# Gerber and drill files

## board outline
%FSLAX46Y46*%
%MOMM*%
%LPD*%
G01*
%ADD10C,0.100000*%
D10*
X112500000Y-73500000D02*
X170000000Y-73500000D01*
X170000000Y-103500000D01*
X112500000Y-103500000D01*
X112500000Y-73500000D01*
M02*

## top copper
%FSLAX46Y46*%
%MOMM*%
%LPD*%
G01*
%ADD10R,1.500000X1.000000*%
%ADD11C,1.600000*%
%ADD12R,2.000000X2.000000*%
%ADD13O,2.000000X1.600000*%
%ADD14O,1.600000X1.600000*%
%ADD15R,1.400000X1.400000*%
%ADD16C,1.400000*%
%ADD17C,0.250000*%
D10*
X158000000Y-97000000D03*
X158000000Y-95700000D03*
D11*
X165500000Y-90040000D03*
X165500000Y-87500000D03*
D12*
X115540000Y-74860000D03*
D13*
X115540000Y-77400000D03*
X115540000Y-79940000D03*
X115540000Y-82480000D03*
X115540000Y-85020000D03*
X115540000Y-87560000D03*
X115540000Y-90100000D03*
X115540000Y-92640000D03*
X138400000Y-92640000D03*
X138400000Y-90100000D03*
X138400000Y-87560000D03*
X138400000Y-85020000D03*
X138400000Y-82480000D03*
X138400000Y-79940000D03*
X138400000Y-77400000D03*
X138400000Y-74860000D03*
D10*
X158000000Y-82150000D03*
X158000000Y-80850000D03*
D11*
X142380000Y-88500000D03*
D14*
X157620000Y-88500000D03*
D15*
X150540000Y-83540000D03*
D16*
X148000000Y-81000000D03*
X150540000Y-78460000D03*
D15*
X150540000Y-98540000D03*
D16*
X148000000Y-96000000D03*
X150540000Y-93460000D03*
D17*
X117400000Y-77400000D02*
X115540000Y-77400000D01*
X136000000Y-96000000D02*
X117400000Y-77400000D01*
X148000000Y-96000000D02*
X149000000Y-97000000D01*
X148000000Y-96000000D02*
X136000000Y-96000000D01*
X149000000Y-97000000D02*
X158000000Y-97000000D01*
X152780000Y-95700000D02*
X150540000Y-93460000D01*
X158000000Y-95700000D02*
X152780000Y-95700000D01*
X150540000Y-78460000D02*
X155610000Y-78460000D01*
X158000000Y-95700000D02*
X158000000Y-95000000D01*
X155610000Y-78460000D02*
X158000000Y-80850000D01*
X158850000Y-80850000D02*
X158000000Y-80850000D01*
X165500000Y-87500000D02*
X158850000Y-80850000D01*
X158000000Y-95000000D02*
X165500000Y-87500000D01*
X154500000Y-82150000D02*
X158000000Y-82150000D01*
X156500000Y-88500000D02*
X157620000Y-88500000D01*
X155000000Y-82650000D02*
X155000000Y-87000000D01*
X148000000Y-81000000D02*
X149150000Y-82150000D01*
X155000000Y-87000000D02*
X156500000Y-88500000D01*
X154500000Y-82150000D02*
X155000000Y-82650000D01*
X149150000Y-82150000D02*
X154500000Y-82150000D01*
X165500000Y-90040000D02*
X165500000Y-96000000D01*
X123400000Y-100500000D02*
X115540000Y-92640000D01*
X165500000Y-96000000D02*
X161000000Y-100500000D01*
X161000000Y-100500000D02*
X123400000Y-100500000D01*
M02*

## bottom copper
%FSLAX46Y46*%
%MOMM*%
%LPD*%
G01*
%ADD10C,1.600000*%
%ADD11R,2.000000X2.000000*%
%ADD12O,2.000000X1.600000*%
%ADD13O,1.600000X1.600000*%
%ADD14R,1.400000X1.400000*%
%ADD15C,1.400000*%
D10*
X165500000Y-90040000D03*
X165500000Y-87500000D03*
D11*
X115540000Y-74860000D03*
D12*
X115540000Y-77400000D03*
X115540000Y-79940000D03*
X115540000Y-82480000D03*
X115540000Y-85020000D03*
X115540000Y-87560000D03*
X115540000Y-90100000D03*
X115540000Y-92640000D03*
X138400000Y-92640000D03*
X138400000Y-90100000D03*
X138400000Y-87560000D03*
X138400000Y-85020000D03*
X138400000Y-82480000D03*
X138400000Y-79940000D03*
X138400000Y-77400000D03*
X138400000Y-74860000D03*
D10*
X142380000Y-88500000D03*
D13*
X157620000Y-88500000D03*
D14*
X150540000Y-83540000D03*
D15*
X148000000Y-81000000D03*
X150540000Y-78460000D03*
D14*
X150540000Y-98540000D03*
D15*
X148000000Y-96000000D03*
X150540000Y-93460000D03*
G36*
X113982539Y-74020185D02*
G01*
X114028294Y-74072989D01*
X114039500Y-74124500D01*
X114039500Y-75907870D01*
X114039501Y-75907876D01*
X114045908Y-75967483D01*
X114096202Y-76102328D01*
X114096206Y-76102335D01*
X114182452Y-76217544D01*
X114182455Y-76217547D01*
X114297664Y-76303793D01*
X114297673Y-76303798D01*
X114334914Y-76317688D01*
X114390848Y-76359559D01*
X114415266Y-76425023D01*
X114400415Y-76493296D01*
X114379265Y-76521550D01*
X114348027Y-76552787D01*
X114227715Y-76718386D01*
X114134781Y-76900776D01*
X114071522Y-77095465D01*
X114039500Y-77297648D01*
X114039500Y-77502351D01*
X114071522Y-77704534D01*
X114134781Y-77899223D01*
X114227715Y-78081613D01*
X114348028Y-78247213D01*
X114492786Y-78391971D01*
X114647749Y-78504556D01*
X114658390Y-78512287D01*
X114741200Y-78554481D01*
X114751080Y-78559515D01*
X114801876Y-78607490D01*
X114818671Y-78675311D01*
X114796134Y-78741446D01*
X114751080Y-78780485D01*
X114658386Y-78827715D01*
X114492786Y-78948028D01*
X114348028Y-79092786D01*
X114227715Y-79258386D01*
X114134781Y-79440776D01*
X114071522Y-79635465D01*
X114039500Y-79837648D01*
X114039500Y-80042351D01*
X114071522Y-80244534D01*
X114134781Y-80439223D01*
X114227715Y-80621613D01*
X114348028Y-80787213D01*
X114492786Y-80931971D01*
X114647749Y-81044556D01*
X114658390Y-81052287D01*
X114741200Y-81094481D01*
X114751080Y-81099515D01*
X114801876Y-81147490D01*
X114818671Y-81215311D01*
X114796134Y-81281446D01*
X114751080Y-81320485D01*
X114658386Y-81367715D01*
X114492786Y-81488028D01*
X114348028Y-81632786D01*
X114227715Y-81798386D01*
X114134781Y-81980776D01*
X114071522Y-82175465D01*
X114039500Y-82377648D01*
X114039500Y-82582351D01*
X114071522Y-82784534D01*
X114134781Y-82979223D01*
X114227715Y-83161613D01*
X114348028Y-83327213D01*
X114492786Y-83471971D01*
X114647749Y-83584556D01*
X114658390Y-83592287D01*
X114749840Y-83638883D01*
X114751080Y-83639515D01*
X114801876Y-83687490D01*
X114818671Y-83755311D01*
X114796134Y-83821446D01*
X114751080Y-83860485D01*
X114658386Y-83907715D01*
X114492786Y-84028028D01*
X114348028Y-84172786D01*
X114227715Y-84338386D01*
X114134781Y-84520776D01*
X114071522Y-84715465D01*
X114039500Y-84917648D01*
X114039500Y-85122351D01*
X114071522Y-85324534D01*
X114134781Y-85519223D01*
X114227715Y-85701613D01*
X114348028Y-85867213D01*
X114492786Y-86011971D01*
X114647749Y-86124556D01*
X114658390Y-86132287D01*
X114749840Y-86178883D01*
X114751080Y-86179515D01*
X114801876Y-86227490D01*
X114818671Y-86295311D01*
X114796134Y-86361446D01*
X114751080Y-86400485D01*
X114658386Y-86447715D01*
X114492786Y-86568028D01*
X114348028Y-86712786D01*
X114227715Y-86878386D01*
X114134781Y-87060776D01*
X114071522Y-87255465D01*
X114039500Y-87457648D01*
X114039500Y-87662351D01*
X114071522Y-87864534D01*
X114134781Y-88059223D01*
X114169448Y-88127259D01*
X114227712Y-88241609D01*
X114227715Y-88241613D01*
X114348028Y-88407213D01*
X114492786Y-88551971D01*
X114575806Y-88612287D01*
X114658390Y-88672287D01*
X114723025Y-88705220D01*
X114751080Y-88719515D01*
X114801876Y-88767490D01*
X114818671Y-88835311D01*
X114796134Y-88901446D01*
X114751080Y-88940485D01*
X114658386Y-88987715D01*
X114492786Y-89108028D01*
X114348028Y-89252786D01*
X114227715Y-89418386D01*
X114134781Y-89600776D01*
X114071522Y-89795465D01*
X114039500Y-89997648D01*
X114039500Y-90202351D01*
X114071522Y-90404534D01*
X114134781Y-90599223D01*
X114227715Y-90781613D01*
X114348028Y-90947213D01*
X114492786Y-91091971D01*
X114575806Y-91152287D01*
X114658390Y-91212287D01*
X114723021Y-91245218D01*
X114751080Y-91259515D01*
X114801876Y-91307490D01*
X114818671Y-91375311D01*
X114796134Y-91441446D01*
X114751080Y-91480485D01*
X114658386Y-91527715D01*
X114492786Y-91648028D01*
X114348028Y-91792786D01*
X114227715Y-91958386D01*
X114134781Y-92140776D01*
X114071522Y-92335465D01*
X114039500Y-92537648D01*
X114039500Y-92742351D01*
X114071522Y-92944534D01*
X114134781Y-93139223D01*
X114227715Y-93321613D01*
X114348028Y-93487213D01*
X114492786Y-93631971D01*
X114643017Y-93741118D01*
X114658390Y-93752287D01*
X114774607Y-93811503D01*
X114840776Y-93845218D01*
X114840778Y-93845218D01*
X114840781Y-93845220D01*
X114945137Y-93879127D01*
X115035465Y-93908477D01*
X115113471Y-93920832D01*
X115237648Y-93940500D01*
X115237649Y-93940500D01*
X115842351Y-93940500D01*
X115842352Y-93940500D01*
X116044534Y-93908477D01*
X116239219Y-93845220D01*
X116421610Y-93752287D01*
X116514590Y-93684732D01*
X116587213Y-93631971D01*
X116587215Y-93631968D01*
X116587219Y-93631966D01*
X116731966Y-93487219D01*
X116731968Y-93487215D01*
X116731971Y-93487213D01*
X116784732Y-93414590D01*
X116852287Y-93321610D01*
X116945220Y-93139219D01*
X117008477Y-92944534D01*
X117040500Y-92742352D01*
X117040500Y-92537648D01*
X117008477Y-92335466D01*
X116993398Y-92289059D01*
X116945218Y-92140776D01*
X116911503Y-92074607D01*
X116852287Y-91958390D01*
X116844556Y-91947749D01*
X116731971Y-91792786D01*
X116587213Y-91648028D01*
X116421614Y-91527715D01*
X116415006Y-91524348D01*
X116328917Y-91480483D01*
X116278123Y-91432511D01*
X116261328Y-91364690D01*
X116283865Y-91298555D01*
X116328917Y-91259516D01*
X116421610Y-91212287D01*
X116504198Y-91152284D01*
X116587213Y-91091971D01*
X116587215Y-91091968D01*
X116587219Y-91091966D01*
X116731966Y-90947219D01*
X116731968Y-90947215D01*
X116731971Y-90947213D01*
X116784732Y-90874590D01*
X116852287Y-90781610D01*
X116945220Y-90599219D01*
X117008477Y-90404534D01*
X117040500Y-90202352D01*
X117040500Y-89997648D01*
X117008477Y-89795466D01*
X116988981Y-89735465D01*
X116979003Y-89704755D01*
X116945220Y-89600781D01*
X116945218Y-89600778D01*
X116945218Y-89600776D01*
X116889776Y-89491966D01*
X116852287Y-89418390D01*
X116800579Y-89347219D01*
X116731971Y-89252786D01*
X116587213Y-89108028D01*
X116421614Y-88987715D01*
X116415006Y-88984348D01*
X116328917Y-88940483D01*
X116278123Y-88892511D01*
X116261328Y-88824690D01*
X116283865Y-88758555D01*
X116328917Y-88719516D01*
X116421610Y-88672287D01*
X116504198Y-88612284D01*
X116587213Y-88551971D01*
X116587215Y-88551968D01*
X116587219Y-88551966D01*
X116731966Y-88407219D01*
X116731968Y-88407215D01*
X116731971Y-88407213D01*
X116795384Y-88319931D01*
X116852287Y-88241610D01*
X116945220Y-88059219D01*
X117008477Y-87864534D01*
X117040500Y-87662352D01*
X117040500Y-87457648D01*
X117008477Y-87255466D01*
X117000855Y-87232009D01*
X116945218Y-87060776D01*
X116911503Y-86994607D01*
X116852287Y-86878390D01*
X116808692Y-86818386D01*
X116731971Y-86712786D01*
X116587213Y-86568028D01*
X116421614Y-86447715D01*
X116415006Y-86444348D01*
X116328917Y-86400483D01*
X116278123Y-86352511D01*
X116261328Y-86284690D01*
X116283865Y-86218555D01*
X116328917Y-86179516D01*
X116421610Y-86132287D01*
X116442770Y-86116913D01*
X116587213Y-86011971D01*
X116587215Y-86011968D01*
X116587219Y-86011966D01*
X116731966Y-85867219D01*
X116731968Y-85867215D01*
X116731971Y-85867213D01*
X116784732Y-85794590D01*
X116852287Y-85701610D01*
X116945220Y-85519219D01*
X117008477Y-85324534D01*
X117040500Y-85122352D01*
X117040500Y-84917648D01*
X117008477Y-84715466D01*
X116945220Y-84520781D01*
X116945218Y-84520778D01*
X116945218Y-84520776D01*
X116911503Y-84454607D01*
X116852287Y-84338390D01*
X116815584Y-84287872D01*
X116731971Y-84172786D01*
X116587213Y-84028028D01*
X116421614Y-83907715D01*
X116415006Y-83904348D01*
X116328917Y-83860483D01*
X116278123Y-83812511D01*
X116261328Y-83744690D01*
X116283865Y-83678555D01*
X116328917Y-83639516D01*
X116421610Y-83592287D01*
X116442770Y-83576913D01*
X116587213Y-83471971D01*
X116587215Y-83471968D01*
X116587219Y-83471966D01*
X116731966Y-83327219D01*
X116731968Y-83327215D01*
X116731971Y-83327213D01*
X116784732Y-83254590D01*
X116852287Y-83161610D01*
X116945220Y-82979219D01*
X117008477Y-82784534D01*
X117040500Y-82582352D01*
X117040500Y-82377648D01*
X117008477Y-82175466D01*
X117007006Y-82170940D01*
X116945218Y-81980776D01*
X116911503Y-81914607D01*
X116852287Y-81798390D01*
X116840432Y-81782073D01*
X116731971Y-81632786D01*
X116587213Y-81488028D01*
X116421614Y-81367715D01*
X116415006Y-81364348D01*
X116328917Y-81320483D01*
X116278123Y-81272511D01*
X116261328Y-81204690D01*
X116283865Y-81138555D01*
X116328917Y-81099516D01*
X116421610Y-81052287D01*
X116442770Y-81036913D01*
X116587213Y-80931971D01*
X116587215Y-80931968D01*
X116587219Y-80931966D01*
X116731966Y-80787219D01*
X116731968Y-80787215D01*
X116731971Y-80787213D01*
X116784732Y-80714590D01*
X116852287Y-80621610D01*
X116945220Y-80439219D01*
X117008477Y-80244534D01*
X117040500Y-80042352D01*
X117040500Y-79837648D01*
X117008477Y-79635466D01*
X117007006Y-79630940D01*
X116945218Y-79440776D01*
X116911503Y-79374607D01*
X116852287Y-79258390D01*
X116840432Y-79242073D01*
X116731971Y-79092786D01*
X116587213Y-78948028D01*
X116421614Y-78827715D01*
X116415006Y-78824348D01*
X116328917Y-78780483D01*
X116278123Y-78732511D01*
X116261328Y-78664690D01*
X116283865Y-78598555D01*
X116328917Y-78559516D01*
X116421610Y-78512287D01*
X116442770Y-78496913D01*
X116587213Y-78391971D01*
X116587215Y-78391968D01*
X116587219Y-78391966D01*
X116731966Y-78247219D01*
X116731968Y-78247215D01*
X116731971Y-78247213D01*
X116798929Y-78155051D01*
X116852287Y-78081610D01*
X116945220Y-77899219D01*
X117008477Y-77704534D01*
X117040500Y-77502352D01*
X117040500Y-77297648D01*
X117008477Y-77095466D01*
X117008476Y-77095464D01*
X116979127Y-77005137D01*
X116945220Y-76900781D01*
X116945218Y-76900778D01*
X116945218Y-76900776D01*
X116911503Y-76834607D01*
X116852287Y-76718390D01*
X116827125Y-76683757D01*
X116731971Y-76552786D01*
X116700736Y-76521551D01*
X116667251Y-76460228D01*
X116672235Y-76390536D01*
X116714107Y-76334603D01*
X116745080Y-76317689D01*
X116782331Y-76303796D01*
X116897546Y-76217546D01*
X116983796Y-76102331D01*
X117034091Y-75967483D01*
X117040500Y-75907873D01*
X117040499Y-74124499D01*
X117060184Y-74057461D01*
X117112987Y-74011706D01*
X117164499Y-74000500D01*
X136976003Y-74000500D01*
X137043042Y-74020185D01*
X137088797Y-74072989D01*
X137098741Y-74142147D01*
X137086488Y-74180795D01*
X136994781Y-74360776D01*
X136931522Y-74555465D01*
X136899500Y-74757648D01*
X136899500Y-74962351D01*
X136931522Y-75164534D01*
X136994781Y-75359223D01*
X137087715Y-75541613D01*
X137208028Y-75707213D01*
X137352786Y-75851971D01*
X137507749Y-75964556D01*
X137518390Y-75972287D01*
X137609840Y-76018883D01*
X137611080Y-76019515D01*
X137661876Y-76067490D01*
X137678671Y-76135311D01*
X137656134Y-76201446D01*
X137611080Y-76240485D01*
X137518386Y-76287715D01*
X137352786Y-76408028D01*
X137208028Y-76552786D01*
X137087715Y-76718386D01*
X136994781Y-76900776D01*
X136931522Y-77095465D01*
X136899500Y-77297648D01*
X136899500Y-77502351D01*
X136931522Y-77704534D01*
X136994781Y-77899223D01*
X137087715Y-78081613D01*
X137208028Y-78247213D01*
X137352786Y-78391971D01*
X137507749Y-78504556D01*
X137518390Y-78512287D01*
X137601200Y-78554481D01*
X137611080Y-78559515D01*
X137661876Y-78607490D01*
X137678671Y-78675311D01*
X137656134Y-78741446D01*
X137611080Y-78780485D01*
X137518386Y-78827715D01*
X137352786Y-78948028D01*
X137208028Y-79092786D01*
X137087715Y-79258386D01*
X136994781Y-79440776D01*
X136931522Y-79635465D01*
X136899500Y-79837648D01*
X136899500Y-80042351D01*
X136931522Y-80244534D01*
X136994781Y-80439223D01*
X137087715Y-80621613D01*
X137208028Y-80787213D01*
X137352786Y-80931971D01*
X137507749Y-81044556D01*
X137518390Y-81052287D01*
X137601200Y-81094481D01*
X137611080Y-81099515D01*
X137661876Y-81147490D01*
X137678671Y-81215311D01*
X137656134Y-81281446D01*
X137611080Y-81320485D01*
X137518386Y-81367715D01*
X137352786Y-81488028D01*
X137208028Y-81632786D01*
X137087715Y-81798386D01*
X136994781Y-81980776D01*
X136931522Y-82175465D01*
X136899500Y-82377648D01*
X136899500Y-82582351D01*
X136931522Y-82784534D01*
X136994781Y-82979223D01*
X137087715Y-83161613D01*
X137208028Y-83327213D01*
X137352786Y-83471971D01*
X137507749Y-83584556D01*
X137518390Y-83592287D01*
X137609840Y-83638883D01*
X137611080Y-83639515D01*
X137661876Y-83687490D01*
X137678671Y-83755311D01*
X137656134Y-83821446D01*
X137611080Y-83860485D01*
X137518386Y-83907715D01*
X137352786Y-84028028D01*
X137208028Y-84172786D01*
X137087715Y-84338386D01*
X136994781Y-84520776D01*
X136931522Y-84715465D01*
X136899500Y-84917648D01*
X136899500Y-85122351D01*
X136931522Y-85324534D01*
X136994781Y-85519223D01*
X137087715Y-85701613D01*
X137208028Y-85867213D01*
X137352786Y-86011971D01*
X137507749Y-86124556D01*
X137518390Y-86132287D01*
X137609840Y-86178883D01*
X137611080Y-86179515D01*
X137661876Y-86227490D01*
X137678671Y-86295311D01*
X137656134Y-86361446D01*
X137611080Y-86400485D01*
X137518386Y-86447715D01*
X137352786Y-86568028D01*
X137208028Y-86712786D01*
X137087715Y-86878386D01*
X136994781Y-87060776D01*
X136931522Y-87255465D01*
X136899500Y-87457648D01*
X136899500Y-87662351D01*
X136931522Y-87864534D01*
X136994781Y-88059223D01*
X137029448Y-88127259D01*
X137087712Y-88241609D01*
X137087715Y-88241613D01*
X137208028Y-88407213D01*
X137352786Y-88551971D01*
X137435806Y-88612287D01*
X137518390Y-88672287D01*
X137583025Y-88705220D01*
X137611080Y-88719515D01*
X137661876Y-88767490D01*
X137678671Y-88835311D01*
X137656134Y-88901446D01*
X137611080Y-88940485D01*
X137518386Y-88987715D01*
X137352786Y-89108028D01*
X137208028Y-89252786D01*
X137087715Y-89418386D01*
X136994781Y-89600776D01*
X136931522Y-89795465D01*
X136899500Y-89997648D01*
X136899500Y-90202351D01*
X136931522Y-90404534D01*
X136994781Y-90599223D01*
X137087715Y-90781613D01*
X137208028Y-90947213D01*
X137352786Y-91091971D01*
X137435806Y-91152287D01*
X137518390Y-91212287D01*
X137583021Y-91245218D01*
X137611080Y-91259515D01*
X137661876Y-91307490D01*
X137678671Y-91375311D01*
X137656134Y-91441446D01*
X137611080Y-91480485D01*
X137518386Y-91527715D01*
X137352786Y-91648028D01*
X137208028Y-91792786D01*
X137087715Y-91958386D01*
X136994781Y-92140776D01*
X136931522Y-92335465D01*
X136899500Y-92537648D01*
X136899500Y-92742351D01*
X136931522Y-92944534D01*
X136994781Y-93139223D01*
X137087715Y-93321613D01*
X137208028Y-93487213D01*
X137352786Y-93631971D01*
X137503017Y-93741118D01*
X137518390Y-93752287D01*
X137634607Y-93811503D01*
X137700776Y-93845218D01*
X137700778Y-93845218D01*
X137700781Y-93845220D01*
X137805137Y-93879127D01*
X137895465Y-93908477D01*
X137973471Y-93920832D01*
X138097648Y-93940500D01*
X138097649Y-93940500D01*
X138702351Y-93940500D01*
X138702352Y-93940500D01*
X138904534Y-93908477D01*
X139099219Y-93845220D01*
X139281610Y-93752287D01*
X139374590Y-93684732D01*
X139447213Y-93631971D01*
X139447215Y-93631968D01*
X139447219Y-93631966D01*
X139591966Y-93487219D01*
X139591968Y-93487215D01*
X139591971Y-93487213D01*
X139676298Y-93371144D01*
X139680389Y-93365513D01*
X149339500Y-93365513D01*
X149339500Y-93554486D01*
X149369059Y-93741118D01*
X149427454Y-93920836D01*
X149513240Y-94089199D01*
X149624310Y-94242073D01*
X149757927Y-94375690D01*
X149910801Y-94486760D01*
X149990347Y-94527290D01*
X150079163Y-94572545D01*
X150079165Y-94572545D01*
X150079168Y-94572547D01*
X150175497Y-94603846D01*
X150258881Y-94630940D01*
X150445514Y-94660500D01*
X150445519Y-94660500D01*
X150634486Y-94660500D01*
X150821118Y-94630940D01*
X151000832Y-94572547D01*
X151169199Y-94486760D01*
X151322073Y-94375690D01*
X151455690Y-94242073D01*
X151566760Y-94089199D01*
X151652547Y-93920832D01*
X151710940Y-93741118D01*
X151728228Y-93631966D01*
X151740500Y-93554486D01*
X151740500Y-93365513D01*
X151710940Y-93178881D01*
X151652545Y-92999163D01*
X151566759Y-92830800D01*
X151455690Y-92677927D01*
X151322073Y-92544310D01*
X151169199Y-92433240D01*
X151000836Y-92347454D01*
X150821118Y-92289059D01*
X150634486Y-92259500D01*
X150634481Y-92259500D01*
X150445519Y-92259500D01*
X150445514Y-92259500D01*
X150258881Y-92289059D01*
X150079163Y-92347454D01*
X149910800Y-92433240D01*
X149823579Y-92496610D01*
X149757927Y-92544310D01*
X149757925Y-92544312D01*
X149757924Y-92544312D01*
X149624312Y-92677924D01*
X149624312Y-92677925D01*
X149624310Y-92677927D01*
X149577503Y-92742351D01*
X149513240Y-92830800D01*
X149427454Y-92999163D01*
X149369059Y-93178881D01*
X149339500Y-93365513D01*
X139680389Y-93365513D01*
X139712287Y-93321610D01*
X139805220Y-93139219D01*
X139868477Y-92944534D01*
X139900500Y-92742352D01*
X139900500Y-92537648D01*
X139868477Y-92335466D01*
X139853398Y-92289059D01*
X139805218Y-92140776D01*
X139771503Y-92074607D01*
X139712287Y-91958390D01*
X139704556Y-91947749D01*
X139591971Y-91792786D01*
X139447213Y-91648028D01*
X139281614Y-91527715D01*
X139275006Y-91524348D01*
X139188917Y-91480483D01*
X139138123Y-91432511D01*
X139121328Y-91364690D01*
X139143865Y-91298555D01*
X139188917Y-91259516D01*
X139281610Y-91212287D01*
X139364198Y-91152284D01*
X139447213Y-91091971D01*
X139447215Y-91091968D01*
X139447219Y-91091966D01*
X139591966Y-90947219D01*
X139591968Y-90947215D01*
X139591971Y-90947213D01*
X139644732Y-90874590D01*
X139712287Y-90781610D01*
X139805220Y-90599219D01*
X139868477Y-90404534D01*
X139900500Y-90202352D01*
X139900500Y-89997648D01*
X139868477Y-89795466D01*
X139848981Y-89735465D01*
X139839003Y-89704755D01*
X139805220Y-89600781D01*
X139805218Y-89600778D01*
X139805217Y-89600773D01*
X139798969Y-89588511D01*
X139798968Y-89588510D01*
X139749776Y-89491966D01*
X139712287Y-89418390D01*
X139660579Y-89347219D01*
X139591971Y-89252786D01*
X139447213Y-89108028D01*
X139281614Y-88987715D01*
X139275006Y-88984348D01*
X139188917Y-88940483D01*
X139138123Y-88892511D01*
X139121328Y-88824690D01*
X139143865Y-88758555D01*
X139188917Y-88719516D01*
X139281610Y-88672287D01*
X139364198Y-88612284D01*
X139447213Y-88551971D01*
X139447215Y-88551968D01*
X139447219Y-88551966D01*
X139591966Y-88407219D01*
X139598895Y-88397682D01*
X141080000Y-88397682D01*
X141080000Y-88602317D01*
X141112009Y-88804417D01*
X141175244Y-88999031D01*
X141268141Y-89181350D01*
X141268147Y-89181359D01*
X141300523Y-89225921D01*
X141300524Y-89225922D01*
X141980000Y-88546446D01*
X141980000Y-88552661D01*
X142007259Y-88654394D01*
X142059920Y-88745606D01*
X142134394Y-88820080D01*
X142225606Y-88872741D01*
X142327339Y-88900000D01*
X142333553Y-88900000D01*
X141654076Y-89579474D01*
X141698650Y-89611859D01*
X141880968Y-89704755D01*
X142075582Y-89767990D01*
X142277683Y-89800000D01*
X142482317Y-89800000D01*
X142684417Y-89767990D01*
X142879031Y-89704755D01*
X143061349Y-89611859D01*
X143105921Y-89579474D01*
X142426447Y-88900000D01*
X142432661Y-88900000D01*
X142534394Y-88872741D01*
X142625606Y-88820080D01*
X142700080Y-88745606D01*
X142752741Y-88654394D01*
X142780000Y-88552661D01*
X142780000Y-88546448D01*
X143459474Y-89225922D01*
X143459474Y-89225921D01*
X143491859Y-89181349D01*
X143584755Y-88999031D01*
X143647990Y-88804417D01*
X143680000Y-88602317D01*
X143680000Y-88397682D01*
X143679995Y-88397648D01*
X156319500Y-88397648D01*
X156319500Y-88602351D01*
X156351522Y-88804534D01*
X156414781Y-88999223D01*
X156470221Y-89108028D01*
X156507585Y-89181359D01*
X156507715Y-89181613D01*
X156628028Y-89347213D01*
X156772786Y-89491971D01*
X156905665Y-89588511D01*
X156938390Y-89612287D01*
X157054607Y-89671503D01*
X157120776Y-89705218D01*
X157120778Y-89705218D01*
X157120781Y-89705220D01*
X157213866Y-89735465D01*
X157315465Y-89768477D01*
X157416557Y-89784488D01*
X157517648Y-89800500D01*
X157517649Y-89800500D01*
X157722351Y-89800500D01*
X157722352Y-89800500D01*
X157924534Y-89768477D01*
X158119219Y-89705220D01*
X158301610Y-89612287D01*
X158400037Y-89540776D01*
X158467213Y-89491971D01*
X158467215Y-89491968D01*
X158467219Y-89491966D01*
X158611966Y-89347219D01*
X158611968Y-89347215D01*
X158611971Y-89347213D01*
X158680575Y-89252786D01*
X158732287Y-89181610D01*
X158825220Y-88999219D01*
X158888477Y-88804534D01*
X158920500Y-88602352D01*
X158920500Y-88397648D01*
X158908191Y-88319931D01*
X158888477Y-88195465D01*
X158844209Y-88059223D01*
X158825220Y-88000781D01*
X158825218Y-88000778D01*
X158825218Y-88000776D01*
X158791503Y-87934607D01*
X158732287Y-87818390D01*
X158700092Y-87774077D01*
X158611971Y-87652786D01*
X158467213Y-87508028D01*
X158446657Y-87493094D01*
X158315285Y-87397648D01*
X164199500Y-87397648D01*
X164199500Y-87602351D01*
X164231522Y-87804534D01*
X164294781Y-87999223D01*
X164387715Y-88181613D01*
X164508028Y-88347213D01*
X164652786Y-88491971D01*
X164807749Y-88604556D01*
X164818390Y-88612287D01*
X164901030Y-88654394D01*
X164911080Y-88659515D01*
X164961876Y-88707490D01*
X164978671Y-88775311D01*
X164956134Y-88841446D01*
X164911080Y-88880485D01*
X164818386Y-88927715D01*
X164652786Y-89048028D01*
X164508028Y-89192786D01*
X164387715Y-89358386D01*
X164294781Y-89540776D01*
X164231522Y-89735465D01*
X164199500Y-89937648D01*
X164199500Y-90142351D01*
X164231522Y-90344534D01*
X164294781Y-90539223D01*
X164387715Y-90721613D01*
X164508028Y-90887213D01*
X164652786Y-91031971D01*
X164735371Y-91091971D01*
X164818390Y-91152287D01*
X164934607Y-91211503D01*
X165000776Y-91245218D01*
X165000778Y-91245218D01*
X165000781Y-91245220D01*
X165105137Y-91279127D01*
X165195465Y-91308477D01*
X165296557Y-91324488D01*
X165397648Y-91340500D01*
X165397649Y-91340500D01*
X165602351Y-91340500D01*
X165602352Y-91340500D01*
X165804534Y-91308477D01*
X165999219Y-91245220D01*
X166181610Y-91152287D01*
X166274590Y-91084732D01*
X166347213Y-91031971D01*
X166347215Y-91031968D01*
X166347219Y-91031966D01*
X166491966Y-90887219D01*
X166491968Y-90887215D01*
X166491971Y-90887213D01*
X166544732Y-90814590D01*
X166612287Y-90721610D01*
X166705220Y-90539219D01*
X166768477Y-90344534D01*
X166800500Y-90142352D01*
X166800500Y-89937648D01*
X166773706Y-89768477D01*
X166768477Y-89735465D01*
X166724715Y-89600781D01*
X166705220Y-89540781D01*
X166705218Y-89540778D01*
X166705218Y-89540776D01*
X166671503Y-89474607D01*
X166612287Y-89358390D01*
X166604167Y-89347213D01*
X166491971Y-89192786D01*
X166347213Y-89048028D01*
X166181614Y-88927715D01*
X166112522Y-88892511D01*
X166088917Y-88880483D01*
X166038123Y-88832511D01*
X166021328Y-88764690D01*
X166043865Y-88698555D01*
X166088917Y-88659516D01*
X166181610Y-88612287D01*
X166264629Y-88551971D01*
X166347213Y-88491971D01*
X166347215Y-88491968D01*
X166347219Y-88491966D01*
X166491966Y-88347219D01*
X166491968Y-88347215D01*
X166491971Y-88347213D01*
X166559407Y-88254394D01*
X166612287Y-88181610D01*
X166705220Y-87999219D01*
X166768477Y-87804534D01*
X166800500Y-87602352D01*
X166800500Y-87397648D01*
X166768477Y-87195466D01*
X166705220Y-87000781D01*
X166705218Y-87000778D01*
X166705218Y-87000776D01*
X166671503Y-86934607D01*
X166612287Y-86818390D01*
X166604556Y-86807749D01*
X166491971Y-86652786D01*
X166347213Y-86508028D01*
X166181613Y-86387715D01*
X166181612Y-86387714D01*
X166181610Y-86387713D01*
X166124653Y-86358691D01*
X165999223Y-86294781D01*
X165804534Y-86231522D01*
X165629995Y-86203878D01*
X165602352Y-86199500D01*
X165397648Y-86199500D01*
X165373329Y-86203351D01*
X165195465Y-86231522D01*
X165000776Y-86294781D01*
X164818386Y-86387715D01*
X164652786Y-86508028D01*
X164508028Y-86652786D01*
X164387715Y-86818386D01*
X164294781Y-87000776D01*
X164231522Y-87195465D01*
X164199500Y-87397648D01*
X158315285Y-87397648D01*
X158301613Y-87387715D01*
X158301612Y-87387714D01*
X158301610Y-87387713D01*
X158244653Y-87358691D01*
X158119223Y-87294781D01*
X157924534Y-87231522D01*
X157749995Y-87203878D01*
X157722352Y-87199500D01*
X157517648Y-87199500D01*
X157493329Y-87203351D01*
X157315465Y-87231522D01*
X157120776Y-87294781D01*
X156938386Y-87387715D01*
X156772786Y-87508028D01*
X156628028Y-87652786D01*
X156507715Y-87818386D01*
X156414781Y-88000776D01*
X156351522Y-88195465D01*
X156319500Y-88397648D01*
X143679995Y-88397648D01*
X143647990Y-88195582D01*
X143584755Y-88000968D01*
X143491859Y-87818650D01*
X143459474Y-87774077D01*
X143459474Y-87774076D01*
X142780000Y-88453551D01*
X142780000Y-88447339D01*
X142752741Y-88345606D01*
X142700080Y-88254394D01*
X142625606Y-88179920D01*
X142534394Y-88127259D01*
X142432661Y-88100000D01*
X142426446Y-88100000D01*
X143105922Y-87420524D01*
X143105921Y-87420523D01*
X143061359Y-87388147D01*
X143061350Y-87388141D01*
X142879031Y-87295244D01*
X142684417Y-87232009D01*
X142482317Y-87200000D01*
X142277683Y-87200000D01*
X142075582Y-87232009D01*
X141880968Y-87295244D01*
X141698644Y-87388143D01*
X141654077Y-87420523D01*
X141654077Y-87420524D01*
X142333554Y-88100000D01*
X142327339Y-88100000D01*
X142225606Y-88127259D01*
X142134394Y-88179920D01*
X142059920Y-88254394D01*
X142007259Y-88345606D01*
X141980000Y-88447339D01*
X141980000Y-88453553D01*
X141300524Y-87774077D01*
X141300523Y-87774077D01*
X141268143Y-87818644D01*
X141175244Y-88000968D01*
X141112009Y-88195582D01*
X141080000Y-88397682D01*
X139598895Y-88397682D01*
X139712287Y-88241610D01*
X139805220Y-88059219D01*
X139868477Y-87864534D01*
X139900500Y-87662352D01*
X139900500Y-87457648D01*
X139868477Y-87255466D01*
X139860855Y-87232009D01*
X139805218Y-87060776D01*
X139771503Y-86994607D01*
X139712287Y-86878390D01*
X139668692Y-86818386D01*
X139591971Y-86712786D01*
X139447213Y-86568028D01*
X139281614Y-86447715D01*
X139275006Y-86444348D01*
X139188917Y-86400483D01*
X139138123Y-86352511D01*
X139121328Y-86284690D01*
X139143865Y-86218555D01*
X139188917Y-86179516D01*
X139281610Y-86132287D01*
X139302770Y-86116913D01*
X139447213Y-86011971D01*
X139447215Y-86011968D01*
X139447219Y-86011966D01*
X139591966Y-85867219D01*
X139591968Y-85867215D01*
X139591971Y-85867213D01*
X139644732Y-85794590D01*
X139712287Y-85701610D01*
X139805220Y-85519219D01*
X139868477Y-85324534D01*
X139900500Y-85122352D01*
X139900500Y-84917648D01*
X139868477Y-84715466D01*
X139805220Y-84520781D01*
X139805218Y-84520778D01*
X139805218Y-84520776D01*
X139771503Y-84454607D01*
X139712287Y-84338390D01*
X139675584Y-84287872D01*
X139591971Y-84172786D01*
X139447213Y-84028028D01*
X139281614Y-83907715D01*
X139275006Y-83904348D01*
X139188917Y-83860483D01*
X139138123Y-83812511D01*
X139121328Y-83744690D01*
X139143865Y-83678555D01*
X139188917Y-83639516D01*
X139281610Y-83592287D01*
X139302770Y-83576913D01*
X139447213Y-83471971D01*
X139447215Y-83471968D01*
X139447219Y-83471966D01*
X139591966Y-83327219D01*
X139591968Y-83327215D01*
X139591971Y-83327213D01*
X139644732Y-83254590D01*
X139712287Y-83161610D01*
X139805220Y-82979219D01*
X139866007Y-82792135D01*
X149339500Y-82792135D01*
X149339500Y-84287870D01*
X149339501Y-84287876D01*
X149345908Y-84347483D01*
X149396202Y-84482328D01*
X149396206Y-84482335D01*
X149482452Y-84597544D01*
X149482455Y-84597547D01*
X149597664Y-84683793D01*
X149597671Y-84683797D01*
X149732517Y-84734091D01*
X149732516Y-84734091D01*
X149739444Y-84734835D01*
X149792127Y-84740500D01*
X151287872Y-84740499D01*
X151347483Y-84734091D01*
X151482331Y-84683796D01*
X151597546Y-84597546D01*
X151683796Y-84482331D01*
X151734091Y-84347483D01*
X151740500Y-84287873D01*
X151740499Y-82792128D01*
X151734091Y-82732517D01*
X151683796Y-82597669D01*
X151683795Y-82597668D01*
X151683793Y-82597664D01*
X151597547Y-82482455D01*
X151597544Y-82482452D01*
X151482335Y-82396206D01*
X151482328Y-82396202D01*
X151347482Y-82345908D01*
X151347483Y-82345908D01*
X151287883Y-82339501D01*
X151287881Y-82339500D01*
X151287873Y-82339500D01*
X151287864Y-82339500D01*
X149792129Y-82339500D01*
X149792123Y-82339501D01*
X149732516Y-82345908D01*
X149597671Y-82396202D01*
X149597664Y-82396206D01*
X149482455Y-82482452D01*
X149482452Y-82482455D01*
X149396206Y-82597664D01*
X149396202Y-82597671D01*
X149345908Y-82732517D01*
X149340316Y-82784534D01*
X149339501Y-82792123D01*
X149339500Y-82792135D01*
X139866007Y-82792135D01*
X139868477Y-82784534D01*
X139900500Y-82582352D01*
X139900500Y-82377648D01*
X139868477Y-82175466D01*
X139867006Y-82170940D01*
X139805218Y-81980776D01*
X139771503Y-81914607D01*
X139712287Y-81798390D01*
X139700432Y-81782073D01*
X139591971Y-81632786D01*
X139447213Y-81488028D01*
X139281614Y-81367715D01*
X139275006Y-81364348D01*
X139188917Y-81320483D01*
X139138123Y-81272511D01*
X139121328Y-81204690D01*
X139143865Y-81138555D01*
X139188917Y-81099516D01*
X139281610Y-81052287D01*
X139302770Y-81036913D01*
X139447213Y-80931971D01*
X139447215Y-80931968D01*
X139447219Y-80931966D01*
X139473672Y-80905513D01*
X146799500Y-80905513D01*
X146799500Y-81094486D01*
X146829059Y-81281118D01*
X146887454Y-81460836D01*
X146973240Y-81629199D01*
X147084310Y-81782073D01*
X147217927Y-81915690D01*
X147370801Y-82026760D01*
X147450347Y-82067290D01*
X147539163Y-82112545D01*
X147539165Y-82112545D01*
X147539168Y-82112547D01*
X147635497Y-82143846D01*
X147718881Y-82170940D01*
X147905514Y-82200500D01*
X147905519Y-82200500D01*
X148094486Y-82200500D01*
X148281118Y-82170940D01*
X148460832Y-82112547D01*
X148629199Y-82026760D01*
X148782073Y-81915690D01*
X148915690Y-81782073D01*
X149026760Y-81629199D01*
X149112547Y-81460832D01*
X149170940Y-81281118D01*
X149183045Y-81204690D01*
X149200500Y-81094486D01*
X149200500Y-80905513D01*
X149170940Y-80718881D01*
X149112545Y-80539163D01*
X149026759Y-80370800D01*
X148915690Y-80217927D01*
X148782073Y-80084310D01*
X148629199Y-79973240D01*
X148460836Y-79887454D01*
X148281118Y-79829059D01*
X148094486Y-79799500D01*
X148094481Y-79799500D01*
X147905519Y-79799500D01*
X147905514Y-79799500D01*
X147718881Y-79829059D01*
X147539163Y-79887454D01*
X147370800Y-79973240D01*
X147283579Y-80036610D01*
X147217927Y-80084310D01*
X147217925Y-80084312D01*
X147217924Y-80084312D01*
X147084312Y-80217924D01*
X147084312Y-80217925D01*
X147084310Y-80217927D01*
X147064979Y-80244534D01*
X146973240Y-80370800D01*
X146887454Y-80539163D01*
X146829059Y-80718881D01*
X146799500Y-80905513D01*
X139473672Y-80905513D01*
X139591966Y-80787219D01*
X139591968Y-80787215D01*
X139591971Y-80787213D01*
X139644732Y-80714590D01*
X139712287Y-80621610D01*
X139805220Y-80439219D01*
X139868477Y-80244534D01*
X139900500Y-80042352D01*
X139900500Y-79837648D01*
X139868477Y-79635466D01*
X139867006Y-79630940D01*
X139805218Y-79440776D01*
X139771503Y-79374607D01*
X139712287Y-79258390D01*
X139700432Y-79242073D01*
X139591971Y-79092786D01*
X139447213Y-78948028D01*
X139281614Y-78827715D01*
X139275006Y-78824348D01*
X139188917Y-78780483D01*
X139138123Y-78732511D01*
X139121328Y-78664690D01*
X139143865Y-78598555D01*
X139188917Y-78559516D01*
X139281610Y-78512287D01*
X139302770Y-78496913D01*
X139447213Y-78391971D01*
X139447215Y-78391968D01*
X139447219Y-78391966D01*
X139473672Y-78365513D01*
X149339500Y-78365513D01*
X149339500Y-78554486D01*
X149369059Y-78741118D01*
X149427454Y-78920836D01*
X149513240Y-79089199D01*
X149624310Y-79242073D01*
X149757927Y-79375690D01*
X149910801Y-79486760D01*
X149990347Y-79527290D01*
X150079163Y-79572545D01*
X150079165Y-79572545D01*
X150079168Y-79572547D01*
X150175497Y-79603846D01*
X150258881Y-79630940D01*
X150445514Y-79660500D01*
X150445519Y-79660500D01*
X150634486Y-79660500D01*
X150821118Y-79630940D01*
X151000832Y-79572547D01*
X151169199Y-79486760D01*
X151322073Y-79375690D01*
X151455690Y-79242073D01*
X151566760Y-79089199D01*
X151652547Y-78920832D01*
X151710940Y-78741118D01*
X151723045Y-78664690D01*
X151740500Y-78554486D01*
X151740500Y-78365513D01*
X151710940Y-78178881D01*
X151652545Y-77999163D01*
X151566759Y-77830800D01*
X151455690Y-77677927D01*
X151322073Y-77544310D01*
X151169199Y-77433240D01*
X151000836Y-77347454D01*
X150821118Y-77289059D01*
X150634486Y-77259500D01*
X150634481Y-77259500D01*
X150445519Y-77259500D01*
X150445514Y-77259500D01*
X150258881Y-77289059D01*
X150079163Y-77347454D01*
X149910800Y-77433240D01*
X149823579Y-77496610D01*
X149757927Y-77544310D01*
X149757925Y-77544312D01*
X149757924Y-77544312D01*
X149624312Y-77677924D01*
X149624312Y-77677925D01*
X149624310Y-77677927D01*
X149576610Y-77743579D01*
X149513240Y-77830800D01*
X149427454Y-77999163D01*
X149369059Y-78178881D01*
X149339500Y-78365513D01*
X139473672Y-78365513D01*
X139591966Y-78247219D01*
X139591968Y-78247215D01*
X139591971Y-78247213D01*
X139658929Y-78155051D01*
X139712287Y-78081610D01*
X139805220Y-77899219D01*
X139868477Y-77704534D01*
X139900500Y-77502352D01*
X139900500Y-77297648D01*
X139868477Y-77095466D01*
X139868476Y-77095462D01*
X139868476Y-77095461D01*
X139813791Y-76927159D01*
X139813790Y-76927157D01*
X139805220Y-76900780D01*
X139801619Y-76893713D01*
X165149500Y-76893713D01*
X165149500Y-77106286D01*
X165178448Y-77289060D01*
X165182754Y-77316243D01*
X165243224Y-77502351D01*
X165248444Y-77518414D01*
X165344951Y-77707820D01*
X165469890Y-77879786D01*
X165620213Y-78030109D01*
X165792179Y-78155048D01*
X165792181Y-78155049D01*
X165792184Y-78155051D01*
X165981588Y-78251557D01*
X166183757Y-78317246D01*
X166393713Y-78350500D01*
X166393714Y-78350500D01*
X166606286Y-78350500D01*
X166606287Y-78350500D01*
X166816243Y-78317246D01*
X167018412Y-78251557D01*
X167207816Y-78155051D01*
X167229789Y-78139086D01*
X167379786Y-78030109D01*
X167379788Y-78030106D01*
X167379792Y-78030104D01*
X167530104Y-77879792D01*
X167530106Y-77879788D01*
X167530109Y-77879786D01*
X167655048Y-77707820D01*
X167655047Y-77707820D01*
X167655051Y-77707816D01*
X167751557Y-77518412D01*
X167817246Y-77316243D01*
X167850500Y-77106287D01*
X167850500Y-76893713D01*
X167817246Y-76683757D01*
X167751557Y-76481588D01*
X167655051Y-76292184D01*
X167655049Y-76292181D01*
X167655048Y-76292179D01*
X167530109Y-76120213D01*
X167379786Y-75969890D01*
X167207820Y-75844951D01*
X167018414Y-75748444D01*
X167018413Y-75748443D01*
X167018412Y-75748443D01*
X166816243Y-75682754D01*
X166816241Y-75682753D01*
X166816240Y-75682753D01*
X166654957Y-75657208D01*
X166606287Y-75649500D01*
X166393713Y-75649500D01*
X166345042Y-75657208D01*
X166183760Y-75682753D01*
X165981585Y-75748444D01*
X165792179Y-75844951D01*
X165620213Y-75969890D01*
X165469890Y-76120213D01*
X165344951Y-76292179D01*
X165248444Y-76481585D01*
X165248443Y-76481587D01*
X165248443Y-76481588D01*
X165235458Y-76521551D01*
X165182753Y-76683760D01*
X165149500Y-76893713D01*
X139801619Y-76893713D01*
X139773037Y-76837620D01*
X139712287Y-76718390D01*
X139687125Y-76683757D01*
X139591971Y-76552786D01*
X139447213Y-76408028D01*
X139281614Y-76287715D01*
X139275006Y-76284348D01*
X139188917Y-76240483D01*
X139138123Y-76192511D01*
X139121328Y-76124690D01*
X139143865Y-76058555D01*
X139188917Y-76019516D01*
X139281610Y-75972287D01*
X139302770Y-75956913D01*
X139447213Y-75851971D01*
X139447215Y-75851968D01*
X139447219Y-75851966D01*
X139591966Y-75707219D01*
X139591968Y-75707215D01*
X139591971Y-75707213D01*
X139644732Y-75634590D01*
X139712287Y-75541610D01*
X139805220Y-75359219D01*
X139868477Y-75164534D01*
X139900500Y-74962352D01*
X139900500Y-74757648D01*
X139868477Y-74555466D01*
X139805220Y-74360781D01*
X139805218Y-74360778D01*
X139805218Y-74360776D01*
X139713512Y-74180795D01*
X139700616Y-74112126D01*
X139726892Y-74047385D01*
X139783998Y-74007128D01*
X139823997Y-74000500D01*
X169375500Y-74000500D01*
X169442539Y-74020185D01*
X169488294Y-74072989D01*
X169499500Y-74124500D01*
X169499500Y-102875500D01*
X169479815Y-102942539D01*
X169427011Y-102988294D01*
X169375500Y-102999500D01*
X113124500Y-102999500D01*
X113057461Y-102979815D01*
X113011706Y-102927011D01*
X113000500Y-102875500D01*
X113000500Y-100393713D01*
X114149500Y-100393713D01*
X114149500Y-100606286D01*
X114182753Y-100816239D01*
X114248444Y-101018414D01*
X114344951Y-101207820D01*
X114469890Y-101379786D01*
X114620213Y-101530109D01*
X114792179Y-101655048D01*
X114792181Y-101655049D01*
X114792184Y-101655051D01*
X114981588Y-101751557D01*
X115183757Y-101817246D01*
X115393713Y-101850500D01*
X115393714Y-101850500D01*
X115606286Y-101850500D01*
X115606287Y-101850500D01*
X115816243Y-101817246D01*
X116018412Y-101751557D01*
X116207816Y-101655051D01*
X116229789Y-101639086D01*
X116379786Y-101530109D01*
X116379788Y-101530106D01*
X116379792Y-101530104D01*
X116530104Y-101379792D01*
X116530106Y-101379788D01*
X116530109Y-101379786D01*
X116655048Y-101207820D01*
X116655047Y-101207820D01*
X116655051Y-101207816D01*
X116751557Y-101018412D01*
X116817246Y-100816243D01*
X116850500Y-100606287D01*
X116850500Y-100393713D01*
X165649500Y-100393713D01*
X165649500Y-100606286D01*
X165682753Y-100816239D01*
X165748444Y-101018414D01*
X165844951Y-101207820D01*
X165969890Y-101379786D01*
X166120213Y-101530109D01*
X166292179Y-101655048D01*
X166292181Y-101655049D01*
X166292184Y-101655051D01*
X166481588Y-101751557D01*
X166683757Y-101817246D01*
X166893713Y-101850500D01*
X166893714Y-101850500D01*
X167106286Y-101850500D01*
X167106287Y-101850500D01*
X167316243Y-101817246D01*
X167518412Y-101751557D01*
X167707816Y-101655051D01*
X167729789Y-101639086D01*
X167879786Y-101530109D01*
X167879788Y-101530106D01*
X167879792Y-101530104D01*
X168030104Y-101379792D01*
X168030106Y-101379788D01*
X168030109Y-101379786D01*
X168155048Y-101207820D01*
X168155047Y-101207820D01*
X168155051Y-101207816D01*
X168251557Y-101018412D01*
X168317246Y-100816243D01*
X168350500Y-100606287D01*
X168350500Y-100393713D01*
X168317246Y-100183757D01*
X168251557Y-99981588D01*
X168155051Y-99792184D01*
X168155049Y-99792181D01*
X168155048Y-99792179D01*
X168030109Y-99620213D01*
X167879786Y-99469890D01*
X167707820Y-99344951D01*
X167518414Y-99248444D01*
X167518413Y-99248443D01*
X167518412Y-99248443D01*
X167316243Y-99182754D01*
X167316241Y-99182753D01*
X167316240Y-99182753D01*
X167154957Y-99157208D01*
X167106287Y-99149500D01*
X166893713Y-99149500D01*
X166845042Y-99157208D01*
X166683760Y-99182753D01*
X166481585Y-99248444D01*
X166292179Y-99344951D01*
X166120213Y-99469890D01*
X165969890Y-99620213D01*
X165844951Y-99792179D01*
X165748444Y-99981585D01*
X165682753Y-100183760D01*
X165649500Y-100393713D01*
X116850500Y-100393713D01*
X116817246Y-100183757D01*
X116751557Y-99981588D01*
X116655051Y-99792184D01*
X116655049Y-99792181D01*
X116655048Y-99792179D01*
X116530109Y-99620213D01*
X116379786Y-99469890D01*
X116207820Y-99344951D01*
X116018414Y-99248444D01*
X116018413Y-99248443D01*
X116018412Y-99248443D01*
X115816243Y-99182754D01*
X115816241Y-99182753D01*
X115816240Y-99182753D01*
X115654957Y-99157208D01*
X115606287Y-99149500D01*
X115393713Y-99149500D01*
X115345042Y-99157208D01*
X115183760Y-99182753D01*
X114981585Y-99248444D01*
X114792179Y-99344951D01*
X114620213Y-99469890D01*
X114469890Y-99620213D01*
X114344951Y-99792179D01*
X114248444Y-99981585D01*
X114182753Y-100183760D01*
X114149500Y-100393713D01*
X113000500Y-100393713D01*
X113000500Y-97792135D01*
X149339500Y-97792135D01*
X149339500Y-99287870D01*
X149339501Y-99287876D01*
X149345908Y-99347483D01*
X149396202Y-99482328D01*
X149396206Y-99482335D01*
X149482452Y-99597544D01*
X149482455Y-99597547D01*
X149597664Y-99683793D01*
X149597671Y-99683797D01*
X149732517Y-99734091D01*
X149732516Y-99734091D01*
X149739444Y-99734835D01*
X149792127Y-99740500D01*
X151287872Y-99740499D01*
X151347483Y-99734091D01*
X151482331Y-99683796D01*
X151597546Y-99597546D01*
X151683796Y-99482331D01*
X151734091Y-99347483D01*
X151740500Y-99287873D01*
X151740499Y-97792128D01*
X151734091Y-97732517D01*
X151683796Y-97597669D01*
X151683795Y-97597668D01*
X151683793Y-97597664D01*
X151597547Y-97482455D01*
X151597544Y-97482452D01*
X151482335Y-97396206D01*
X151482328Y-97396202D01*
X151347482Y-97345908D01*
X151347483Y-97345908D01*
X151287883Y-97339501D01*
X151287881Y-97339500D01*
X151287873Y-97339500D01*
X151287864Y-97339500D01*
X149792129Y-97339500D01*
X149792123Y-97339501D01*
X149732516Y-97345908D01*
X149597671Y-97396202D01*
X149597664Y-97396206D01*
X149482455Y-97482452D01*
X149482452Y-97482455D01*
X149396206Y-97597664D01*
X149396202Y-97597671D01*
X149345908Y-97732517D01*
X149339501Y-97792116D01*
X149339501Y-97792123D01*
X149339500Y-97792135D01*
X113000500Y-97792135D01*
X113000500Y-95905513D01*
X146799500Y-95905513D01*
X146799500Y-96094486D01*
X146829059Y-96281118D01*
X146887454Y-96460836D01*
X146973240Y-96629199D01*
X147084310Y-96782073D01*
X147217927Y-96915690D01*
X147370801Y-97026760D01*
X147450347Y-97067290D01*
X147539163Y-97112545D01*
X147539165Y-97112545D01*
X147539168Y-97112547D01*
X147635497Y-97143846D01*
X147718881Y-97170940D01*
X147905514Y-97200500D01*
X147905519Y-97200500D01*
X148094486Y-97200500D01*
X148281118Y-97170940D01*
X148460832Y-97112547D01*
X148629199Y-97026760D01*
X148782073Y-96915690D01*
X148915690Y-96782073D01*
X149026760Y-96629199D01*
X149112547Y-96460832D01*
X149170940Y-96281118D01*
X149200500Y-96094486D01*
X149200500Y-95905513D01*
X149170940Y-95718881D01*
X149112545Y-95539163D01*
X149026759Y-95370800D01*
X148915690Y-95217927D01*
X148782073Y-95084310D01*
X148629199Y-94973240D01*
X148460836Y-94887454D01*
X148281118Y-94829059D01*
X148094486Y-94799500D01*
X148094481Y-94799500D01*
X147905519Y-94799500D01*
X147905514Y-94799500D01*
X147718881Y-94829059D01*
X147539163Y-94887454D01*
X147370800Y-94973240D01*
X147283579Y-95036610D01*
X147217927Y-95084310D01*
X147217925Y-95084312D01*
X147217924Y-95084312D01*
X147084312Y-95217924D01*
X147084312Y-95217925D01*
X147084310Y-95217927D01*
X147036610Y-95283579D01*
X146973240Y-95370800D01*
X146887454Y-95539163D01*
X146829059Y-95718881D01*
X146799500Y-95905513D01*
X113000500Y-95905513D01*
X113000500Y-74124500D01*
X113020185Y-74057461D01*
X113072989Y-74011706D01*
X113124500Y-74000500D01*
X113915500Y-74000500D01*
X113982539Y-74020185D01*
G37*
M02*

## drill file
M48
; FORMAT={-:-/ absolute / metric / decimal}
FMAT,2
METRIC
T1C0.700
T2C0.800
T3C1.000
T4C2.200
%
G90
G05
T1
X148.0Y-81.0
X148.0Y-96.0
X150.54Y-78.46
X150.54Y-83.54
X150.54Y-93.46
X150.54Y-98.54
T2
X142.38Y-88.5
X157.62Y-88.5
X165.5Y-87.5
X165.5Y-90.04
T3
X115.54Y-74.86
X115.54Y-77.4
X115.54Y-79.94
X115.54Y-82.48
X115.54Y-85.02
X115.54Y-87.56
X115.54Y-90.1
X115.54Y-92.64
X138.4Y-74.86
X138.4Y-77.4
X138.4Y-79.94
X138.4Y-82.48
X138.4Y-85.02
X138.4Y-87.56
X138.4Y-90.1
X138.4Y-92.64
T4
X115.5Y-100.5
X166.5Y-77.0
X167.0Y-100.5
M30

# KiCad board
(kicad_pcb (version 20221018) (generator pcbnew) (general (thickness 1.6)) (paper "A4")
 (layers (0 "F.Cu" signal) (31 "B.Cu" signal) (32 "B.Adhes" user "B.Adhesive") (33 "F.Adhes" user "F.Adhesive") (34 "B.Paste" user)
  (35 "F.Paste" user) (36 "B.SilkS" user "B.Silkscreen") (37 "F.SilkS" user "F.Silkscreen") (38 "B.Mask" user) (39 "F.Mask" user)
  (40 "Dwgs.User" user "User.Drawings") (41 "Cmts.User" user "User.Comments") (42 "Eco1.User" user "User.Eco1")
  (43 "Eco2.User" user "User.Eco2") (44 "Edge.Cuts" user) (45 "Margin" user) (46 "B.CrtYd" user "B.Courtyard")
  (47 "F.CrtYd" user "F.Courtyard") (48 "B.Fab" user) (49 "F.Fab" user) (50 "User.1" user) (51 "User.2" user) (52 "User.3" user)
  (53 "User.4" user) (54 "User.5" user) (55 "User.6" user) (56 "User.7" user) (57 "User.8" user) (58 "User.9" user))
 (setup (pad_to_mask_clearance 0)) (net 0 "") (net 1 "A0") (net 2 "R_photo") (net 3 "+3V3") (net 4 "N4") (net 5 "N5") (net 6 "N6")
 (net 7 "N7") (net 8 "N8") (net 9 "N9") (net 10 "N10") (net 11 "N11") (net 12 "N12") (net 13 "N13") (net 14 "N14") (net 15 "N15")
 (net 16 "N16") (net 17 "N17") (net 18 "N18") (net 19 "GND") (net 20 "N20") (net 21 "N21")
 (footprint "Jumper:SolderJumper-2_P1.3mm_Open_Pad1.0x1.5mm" (layer "F.Cu") (at 158 96.35 90)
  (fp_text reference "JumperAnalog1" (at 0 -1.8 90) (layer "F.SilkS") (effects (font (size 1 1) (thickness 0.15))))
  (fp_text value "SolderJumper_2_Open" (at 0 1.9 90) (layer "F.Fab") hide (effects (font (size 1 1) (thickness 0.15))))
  (pad "1" smd rect (at -0.65 0 90) (size 1 1.5) (layers "F.Cu" "F.Mask") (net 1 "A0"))
  (pad "2" smd rect (at 0.65 0 90) (size 1 1.5) (layers "F.Cu" "F.Mask") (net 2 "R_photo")))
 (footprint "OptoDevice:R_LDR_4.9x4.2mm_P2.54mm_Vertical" (layer "F.Cu") (at 165.5 90.04 90)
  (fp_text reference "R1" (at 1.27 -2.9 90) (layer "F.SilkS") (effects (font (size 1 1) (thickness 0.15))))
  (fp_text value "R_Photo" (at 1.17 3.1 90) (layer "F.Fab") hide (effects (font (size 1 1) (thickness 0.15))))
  (pad "1" thru_hole circle (at 0 0 90) (size 1.6 1.6) (drill 0.8) (layers "*.Cu" "*.Mask") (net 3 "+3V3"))
  (pad "2" thru_hole circle (at 2.54 0 90) (size 1.6 1.6) (drill 0.8) (layers "*.Cu" "*.Mask") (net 2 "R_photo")))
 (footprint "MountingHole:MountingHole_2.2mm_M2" (layer "F.Cu") (at 115.5 100.5)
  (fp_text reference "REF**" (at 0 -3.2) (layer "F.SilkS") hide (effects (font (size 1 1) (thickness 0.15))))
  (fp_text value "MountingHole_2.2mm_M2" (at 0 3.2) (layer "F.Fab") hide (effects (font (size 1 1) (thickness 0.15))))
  (pad "" np_thru_hole circle (at 0 0) (size 2.2 2.2) (drill 2.2) (layers "*.Cu" "*.Mask")))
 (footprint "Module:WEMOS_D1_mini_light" (layer "F.Cu") (at 115.54 74.86)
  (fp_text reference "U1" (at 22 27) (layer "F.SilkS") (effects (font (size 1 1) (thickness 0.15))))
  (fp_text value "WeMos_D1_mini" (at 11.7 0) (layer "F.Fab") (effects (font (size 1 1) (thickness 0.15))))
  (pad "1" thru_hole rect (at 0 0) (size 2 2) (drill 1) (layers "*.Cu" "*.Mask") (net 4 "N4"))
  (pad "2" thru_hole oval (at 0 2.54) (size 2 1.6) (drill 1) (layers "*.Cu" "*.Mask") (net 1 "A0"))
  (pad "3" thru_hole oval (at 0 5.08) (size 2 1.6) (drill 1) (layers "*.Cu" "*.Mask") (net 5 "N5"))
  (pad "4" thru_hole oval (at 0 7.62) (size 2 1.6) (drill 1) (layers "*.Cu" "*.Mask") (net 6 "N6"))
  (pad "5" thru_hole oval (at 0 10.16) (size 2 1.6) (drill 1) (layers "*.Cu" "*.Mask") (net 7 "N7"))
  (pad "6" thru_hole oval (at 0 12.7) (size 2 1.6) (drill 1) (layers "*.Cu" "*.Mask") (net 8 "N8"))
  (pad "7" thru_hole oval (at 0 15.24) (size 2 1.6) (drill 1) (layers "*.Cu" "*.Mask") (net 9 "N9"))
  (pad "8" thru_hole oval (at 0 17.78) (size 2 1.6) (drill 1) (layers "*.Cu" "*.Mask") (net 3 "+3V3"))
  (pad "9" thru_hole oval (at 22.86 17.78) (size 2 1.6) (drill 1) (layers "*.Cu" "*.Mask") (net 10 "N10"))
  (pad "10" thru_hole oval (at 22.86 15.24) (size 2 1.6) (drill 1) (layers "*.Cu" "*.Mask") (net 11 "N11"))
  (pad "11" thru_hole oval (at 22.86 12.7) (size 2 1.6) (drill 1) (layers "*.Cu" "*.Mask") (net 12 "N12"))
  (pad "12" thru_hole oval (at 22.86 10.16) (size 2 1.6) (drill 1) (layers "*.Cu" "*.Mask") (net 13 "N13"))
  (pad "13" thru_hole oval (at 22.86 7.62) (size 2 1.6) (drill 1) (layers "*.Cu" "*.Mask") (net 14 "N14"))
  (pad "14" thru_hole oval (at 22.86 5.08) (size 2 1.6) (drill 1) (layers "*.Cu" "*.Mask") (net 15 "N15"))
  (pad "15" thru_hole oval (at 22.86 2.54) (size 2 1.6) (drill 1) (layers "*.Cu" "*.Mask") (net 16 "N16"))
  (pad "16" thru_hole oval (at 22.86 0) (size 2 1.6) (drill 1) (layers "*.Cu" "*.Mask") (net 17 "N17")))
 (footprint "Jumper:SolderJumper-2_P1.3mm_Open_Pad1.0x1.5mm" (layer "F.Cu") (at 158 81.5 90)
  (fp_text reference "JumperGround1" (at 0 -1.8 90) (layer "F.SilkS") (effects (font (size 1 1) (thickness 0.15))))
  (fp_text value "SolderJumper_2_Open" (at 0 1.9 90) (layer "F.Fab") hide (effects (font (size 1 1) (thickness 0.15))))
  (pad "1" smd rect (at -0.65 0 90) (size 1 1.5) (layers "F.Cu" "F.Mask") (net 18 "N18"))
  (pad "2" smd rect (at 0.65 0 90) (size 1 1.5) (layers "F.Cu" "F.Mask") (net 2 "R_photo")))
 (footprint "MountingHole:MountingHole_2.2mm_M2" (layer "F.Cu") (at 166.5 77)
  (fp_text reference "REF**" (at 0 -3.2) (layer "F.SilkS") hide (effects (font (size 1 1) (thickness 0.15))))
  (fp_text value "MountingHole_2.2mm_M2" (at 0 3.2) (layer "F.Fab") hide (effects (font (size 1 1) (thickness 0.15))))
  (pad "" np_thru_hole circle (at 0 0) (size 2.2 2.2) (drill 2.2) (layers "*.Cu" "*.Mask")))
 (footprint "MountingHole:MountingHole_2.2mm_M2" (layer "F.Cu") (at 167 100.5)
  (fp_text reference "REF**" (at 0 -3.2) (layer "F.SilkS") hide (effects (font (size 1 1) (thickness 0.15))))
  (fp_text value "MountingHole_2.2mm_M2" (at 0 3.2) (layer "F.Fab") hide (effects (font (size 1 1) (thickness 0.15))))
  (pad "" np_thru_hole circle (at 0 0) (size 2.2 2.2) (drill 2.2) (layers "*.Cu" "*.Mask")))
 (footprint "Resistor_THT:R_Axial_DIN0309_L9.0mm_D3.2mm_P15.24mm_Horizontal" (layer "F.Cu") (at 142.38 88.5)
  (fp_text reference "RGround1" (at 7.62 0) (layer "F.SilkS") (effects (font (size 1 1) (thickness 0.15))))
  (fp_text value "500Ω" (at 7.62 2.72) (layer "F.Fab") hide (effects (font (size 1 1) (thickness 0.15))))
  (pad "1" thru_hole circle (at 0 0) (size 1.6 1.6) (drill 0.8) (layers "*.Cu" "*.Mask") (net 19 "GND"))
  (pad "2" thru_hole oval (at 15.24 0) (size 1.6 1.6) (drill 0.8) (layers "*.Cu" "*.Mask") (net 18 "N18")))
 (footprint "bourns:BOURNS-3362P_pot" (layer "F.Cu") (at 150.54 81 90)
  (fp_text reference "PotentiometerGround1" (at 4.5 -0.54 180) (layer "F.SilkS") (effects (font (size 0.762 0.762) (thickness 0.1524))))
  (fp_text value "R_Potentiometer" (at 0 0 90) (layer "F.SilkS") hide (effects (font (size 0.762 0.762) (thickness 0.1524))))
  (pad "1" thru_hole rect (at -2.54 0 90) (size 1.4 1.4) (drill 0.7) (layers "*.Cu" "*.Mask" "F.SilkS") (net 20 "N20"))
  (pad "2" thru_hole circle (at 0 -2.54 90) (size 1.4 1.4) (drill 0.7) (layers "*.Cu" "*.Mask" "F.SilkS") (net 18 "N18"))
  (pad "3" thru_hole circle (at 2.54 0 90) (size 1.4 1.4) (drill 0.7) (layers "*.Cu" "*.Mask" "F.SilkS") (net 2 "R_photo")))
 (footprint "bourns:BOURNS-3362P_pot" (layer "F.Cu") (at 150.54 96 90)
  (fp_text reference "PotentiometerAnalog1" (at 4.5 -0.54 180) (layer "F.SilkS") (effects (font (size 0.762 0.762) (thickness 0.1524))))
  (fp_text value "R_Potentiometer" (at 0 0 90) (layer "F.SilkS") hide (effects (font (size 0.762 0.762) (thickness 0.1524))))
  (pad "1" thru_hole rect (at -2.54 0 90) (size 1.4 1.4) (drill 0.7) (layers "*.Cu" "*.Mask" "F.SilkS") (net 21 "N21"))
  (pad "2" thru_hole circle (at 0 -2.54 90) (size 1.4 1.4) (drill 0.7) (layers "*.Cu" "*.Mask" "F.SilkS") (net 1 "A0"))
  (pad "3" thru_hole circle (at 2.54 0 90) (size 1.4 1.4) (drill 0.7) (layers "*.Cu" "*.Mask" "F.SilkS") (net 2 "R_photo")))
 (gr_rect (start 112.5 73.5) (end 170 103.5) (stroke (width 0.1) (type default)) (fill none) (layer "Edge.Cuts"))
 (segment (start 117.4 77.4) (end 115.54 77.4) (width 0.25) (layer "F.Cu") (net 1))
 (segment (start 136 96) (end 117.4 77.4) (width 0.25) (layer "F.Cu") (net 1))
 (segment (start 148 96) (end 149 97) (width 0.25) (layer "F.Cu") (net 1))
 (segment (start 148 96) (end 136 96) (width 0.25) (layer "F.Cu") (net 1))
 (segment (start 149 97) (end 158 97) (width 0.25) (layer "F.Cu") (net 1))
 (segment (start 152.78 95.7) (end 150.54 93.46) (width 0.25) (layer "F.Cu") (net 2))
 (segment (start 158 95.7) (end 152.78 95.7) (width 0.25) (layer "F.Cu") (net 2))
 (segment (start 150.54 78.46) (end 155.61 78.46) (width 0.25) (layer "F.Cu") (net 2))
 (segment (start 158 95.7) (end 158 95) (width 0.25) (layer "F.Cu") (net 2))
 (segment (start 155.61 78.46) (end 158 80.85) (width 0.25) (layer "F.Cu") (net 2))
 (segment (start 158.85 80.85) (end 158 80.85) (width 0.25) (layer "F.Cu") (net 2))
 (segment (start 165.5 87.5) (end 158.85 80.85) (width 0.25) (layer "F.Cu") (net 2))
 (segment (start 158 95) (end 165.5 87.5) (width 0.25) (layer "F.Cu") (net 2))
 (segment (start 154.5 82.15) (end 158 82.15) (width 0.25) (layer "F.Cu") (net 18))
 (segment (start 156.5 88.5) (end 157.62 88.5) (width 0.25) (layer "F.Cu") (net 18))
 (segment (start 155 82.65) (end 155 87) (width 0.25) (layer "F.Cu") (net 18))
 (segment (start 148 81) (end 149.15 82.15) (width 0.25) (layer "F.Cu") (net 18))
 (segment (start 155 87) (end 156.5 88.5) (width 0.25) (layer "F.Cu") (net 18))
 (segment (start 154.5 82.15) (end 155 82.65) (width 0.25) (layer "F.Cu") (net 18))
 (segment (start 149.15 82.15) (end 154.5 82.15) (width 0.25) (layer "F.Cu") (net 18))
 (segment (start 165.5 90.04) (end 165.5 96) (width 0.25) (layer "F.Cu") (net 3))
 (segment (start 123.4 100.5) (end 115.54 92.64) (width 0.25) (layer "F.Cu") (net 3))
 (segment (start 165.5 96) (end 161 100.5) (width 0.25) (layer "F.Cu") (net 3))
 (segment (start 161 100.5) (end 123.4 100.5) (width 0.25) (layer "F.Cu") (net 3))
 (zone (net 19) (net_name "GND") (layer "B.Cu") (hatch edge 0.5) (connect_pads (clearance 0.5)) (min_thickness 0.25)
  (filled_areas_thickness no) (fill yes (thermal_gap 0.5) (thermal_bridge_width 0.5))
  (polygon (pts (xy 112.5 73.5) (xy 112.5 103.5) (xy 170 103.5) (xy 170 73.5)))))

